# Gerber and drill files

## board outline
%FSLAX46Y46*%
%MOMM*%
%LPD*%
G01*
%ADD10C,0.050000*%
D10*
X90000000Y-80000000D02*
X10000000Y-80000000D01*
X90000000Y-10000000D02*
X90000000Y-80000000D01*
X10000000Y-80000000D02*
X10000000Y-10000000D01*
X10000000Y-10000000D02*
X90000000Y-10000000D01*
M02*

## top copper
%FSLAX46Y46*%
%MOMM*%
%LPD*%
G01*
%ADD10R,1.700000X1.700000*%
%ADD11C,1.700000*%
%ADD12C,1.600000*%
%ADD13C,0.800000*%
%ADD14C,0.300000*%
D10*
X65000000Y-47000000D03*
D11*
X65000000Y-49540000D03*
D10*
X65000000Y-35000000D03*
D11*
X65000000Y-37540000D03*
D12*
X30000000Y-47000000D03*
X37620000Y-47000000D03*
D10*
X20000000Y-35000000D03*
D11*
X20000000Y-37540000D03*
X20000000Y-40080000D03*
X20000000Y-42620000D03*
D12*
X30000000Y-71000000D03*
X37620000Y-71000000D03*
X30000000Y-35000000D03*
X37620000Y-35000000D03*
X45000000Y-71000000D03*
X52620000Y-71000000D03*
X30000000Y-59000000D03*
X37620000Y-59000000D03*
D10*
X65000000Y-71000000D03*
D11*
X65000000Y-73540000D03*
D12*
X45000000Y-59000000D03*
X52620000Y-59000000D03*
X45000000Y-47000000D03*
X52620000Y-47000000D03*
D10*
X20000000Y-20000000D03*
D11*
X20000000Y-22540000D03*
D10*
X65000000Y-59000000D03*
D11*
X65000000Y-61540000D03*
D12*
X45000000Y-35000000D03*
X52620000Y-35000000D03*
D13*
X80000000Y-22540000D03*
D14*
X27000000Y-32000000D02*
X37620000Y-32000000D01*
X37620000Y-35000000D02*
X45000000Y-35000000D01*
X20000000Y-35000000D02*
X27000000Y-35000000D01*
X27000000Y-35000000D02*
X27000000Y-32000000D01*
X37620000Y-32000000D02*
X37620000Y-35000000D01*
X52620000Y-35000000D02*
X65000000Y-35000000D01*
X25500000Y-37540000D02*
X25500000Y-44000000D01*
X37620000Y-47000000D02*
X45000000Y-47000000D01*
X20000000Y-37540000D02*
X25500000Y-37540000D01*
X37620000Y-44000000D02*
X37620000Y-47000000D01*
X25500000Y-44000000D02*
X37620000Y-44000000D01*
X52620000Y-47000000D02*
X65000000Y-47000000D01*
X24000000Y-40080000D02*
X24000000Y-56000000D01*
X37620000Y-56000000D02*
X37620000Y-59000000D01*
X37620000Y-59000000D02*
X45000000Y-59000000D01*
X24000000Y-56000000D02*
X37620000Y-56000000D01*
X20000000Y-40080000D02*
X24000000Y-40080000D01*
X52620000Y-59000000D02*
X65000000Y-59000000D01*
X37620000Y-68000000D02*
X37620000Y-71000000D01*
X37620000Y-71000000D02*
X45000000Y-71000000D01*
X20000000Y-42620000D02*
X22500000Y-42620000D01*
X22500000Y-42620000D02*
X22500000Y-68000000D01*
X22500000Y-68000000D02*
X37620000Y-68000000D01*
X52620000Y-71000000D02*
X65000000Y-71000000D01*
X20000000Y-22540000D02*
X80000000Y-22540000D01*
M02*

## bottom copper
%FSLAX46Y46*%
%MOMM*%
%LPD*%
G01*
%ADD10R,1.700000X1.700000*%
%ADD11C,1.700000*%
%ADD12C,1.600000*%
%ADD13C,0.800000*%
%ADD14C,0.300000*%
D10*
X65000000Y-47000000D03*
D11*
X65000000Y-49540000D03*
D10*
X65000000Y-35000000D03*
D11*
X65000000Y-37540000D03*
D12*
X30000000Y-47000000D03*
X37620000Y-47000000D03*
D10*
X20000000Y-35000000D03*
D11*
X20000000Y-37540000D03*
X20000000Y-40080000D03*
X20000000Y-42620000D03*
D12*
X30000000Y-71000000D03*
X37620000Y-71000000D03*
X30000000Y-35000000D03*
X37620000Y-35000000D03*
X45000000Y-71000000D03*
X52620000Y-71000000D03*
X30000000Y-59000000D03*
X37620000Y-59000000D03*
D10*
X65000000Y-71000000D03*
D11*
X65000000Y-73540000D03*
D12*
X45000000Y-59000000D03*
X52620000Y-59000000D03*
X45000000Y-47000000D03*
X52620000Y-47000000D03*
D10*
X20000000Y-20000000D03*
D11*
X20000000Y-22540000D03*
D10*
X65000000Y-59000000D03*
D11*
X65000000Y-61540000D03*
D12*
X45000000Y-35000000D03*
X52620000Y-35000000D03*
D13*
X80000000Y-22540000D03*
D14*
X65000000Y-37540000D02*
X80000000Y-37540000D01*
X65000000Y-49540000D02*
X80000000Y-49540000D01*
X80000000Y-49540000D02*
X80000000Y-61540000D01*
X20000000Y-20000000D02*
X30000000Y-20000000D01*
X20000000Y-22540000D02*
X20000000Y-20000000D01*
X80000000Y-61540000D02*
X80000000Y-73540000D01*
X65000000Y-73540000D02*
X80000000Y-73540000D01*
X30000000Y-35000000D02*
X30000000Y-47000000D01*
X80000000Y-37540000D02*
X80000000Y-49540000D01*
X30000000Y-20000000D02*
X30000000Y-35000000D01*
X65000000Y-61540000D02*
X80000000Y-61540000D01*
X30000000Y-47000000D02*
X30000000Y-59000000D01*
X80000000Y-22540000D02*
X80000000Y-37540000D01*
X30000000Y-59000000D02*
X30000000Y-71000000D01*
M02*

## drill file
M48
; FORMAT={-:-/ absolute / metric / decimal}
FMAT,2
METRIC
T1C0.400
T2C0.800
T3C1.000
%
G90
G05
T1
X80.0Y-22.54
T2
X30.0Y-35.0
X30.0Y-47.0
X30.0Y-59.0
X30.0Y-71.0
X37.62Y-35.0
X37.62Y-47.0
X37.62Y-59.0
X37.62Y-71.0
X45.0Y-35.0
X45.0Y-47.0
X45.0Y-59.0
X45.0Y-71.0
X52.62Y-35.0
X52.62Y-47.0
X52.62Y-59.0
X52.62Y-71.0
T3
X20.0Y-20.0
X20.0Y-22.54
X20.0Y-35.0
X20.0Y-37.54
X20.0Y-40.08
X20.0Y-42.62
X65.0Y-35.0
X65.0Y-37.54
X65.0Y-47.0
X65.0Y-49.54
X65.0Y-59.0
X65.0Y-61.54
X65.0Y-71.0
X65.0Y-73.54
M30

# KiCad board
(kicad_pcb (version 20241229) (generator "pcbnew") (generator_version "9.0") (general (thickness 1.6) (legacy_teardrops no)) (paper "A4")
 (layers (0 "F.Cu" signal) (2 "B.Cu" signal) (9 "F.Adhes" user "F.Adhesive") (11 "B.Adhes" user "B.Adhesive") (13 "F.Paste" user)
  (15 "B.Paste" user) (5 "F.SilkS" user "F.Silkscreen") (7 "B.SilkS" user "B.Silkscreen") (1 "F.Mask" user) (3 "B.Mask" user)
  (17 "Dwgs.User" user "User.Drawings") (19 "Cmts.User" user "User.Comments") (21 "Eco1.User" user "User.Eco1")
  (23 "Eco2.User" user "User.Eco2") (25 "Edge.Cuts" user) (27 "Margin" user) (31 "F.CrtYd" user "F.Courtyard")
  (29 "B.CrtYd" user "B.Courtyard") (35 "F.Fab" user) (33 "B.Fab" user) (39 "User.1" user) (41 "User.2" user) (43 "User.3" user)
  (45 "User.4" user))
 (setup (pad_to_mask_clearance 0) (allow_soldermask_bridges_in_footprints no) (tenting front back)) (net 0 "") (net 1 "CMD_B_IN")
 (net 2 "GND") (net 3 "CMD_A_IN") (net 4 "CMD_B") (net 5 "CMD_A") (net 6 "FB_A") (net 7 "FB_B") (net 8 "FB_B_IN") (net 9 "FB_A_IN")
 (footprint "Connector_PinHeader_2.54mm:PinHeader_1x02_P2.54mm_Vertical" (layer "F.Cu") (at 65 47)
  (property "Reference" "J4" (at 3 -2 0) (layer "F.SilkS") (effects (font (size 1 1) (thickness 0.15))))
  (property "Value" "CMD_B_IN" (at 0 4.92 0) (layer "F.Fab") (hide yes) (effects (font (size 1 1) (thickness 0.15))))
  (pad "1" thru_hole rect (at 0 0) (size 1.7 1.7) (drill 1) (layers "*.Cu" "*.Mask") (remove_unused_layers no) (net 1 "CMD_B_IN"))
  (pad "2" thru_hole circle (at 0 2.54) (size 1.7 1.7) (drill 1) (layers "*.Cu" "*.Mask") (remove_unused_layers no) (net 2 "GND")))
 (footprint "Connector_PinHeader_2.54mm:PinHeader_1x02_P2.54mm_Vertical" (layer "F.Cu") (at 65 35)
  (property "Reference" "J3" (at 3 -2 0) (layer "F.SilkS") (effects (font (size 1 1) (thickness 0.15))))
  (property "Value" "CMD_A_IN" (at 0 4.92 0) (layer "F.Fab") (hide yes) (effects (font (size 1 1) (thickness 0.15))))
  (pad "1" thru_hole rect (at 0 0) (size 1.7 1.7) (drill 1) (layers "*.Cu" "*.Mask") (remove_unused_layers no) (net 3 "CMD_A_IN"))
  (pad "2" thru_hole circle (at 0 2.54) (size 1.7 1.7) (drill 1) (layers "*.Cu" "*.Mask") (remove_unused_layers no) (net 2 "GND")))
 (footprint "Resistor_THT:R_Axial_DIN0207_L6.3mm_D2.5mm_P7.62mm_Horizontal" (layer "F.Cu") (at 30 47)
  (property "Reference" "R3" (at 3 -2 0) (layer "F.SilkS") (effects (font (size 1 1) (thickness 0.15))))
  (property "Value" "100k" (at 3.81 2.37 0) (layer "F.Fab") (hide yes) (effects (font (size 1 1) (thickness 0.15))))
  (pad "1" thru_hole circle (at 0 0) (size 1.6 1.6) (drill 0.8) (layers "*.Cu" "*.Mask") (remove_unused_layers no) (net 2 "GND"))
  (pad "2" thru_hole circle (at 7.62 0) (size 1.6 1.6) (drill 0.8) (layers "*.Cu" "*.Mask") (remove_unused_layers no) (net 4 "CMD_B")))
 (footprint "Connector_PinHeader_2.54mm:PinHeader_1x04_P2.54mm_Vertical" (layer "F.Cu") (at 20 35)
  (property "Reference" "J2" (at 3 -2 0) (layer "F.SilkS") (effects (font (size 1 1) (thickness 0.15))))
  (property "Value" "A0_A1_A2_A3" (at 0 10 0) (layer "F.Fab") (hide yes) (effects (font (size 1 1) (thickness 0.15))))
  (pad "1" thru_hole rect (at 0 0) (size 1.7 1.7) (drill 1) (layers "*.Cu" "*.Mask") (remove_unused_layers no) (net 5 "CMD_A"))
  (pad "2" thru_hole circle (at 0 2.54) (size 1.7 1.7) (drill 1) (layers "*.Cu" "*.Mask") (remove_unused_layers no) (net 4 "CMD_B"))
  (pad "3" thru_hole circle (at 0 5.08) (size 1.7 1.7) (drill 1) (layers "*.Cu" "*.Mask") (remove_unused_layers no) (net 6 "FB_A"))
  (pad "4" thru_hole circle (at 0 7.62) (size 1.7 1.7) (drill 1) (layers "*.Cu" "*.Mask") (remove_unused_layers no) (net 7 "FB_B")))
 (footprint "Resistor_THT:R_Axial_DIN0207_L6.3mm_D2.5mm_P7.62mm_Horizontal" (layer "F.Cu") (at 30 71)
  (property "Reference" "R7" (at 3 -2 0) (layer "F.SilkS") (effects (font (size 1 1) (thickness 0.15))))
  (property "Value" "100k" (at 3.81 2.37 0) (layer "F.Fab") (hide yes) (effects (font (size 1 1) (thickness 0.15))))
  (pad "1" thru_hole circle (at 0 0) (size 1.6 1.6) (drill 0.8) (layers "*.Cu" "*.Mask") (remove_unused_layers no) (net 2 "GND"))
  (pad "2" thru_hole circle (at 7.62 0) (size 1.6 1.6) (drill 0.8) (layers "*.Cu" "*.Mask") (remove_unused_layers no) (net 7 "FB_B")))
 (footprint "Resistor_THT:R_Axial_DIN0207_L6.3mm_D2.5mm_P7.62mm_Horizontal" (layer "F.Cu") (at 30 35)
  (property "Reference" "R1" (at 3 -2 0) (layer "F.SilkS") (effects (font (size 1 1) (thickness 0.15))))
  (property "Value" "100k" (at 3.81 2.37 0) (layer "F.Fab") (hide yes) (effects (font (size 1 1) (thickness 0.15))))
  (pad "1" thru_hole circle (at 0 0) (size 1.6 1.6) (drill 0.8) (layers "*.Cu" "*.Mask") (remove_unused_layers no) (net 2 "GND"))
  (pad "2" thru_hole circle (at 7.62 0) (size 1.6 1.6) (drill 0.8) (layers "*.Cu" "*.Mask") (remove_unused_layers no) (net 5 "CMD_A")))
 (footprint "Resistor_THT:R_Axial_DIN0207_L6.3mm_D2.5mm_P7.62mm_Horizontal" (layer "F.Cu") (at 45 71)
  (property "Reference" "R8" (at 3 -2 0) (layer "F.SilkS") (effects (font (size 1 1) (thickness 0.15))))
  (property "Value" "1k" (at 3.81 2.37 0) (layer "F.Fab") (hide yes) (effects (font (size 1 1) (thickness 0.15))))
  (pad "1" thru_hole circle (at 0 0) (size 1.6 1.6) (drill 0.8) (layers "*.Cu" "*.Mask") (remove_unused_layers no) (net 7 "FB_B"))
  (pad "2" thru_hole circle (at 7.62 0) (size 1.6 1.6) (drill 0.8) (layers "*.Cu" "*.Mask") (remove_unused_layers no) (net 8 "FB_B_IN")))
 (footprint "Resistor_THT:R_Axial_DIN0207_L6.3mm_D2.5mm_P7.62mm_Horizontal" (layer "F.Cu") (at 30 59)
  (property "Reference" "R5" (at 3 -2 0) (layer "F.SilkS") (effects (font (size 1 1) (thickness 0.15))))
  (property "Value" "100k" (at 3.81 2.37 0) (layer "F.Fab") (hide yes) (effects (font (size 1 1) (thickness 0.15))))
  (pad "1" thru_hole circle (at 0 0) (size 1.6 1.6) (drill 0.8) (layers "*.Cu" "*.Mask") (remove_unused_layers no) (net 2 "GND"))
  (pad "2" thru_hole circle (at 7.62 0) (size 1.6 1.6) (drill 0.8) (layers "*.Cu" "*.Mask") (remove_unused_layers no) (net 6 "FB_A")))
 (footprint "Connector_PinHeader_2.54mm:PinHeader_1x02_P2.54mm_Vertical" (layer "F.Cu") (at 65 71)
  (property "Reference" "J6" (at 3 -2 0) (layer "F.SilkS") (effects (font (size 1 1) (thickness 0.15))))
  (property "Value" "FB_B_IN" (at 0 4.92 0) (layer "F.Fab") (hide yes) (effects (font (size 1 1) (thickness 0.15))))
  (pad "1" thru_hole rect (at 0 0) (size 1.7 1.7) (drill 1) (layers "*.Cu" "*.Mask") (remove_unused_layers no) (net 8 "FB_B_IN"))
  (pad "2" thru_hole circle (at 0 2.54) (size 1.7 1.7) (drill 1) (layers "*.Cu" "*.Mask") (remove_unused_layers no) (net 2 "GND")))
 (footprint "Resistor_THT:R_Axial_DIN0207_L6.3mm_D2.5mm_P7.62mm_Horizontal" (layer "F.Cu") (at 45 59)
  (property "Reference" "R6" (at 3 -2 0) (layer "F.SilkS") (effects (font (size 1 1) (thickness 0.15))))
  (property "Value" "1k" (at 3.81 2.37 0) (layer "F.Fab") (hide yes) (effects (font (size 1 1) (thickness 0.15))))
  (pad "1" thru_hole circle (at 0 0) (size 1.6 1.6) (drill 0.8) (layers "*.Cu" "*.Mask") (remove_unused_layers no) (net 6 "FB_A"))
  (pad "2" thru_hole circle (at 7.62 0) (size 1.6 1.6) (drill 0.8) (layers "*.Cu" "*.Mask") (remove_unused_layers no) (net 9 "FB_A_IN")))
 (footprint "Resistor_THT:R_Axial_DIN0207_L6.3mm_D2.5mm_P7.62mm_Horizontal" (layer "F.Cu") (at 45 47)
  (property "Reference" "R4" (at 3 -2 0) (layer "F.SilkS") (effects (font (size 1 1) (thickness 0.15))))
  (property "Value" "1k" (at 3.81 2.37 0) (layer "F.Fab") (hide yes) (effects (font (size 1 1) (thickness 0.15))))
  (pad "1" thru_hole circle (at 0 0) (size 1.6 1.6) (drill 0.8) (layers "*.Cu" "*.Mask") (remove_unused_layers no) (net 4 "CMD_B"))
  (pad "2" thru_hole circle (at 7.62 0) (size 1.6 1.6) (drill 0.8) (layers "*.Cu" "*.Mask") (remove_unused_layers no) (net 1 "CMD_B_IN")))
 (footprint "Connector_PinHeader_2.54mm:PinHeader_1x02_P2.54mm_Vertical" (layer "F.Cu") (at 20 20)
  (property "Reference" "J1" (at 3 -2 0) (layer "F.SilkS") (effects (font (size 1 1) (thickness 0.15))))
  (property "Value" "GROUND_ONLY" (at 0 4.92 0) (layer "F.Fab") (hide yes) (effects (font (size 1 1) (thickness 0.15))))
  (pad "1" thru_hole rect (at 0 0) (size 1.7 1.7) (drill 1) (layers "*.Cu" "*.Mask") (remove_unused_layers no) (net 2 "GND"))
  (pad "2" thru_hole circle (at 0 2.54) (size 1.7 1.7) (drill 1) (layers "*.Cu" "*.Mask") (remove_unused_layers no) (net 2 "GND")))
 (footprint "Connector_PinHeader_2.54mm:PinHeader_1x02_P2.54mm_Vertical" (layer "F.Cu") (at 65 59)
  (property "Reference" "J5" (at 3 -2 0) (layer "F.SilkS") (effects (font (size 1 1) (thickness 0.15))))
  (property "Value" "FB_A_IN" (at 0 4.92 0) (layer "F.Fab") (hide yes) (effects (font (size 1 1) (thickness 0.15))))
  (pad "1" thru_hole rect (at 0 0) (size 1.7 1.7) (drill 1) (layers "*.Cu" "*.Mask") (remove_unused_layers no) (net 9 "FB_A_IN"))
  (pad "2" thru_hole circle (at 0 2.54) (size 1.7 1.7) (drill 1) (layers "*.Cu" "*.Mask") (remove_unused_layers no) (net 2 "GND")))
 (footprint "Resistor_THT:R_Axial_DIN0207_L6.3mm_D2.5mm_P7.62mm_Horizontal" (layer "F.Cu") (at 45 35)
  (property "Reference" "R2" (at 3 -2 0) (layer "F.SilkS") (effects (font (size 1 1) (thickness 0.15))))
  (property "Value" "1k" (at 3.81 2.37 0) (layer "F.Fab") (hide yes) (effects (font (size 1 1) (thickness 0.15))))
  (pad "1" thru_hole circle (at 0 0) (size 1.6 1.6) (drill 0.8) (layers "*.Cu" "*.Mask") (remove_unused_layers no) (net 5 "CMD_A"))
  (pad "2" thru_hole circle (at 7.62 0) (size 1.6 1.6) (drill 0.8) (layers "*.Cu" "*.Mask") (remove_unused_layers no) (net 3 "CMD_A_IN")))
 (gr_line (start 90 80) (end 10 80) (stroke (width 0.05) (type default)) (layer "Edge.Cuts"))
 (gr_line (start 90 10) (end 90 80) (stroke (width 0.05) (type default)) (layer "Edge.Cuts"))
 (gr_line (start 10 80) (end 10 10) (stroke (width 0.05) (type default)) (layer "Edge.Cuts"))
 (gr_line (start 10 10) (end 90 10) (stroke (width 0.05) (type default)) (layer "Edge.Cuts"))
 (segment (start 27 32) (end 37.62 32) (width 0.3) (layer "F.Cu") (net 5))
 (segment (start 37.62 35) (end 45 35) (width 0.3) (layer "F.Cu") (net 5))
 (segment (start 20 35) (end 27 35) (width 0.3) (layer "F.Cu") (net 5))
 (segment (start 27 35) (end 27 32) (width 0.3) (layer "F.Cu") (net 5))
 (segment (start 37.62 32) (end 37.62 35) (width 0.3) (layer "F.Cu") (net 5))
 (segment (start 52.62 35) (end 65 35) (width 0.3) (layer "F.Cu") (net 3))
 (segment (start 25.5 37.54) (end 25.5 44) (width 0.3) (layer "F.Cu") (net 4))
 (segment (start 37.62 47) (end 45 47) (width 0.3) (layer "F.Cu") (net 4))
 (segment (start 20 37.54) (end 25.5 37.54) (width 0.3) (layer "F.Cu") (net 4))
 (segment (start 37.62 44) (end 37.62 47) (width 0.3) (layer "F.Cu") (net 4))
 (segment (start 25.5 44) (end 37.62 44) (width 0.3) (layer "F.Cu") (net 4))
 (segment (start 52.62 47) (end 65 47) (width 0.3) (layer "F.Cu") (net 1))
 (segment (start 24 40.08) (end 24 56) (width 0.3) (layer "F.Cu") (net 6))
 (segment (start 37.62 56) (end 37.62 59) (width 0.3) (layer "F.Cu") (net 6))
 (segment (start 37.62 59) (end 45 59) (width 0.3) (layer "F.Cu") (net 6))
 (segment (start 24 56) (end 37.62 56) (width 0.3) (layer "F.Cu") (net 6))
 (segment (start 20 40.08) (end 24 40.08) (width 0.3) (layer "F.Cu") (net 6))
 (segment (start 52.62 59) (end 65 59) (width 0.3) (layer "F.Cu") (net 9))
 (segment (start 37.62 68) (end 37.62 71) (width 0.3) (layer "F.Cu") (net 7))
 (segment (start 37.62 71) (end 45 71) (width 0.3) (layer "F.Cu") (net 7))
 (segment (start 20 42.62) (end 22.5 42.62) (width 0.3) (layer "F.Cu") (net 7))
 (segment (start 22.5 42.62) (end 22.5 68) (width 0.3) (layer "F.Cu") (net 7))
 (segment (start 22.5 68) (end 37.62 68) (width 0.3) (layer "F.Cu") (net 7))
 (segment (start 52.62 71) (end 65 71) (width 0.3) (layer "F.Cu") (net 8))
 (segment (start 20 22.54) (end 80 22.54) (width 0.3) (layer "F.Cu") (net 2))
 (via (at 80 22.54) (size 0.8) (drill 0.4) (layers "F.Cu" "B.Cu") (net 2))
 (segment (start 65 37.54) (end 80 37.54) (width 0.3) (layer "B.Cu") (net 2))
 (segment (start 65 49.54) (end 80 49.54) (width 0.3) (layer "B.Cu") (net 2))
 (segment (start 80 49.54) (end 80 61.54) (width 0.3) (layer "B.Cu") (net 2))
 (segment (start 20 20) (end 30 20) (width 0.3) (layer "B.Cu") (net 2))
 (segment (start 20 22.54) (end 20 20) (width 0.3) (layer "B.Cu") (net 2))
 (segment (start 80 61.54) (end 80 73.54) (width 0.3) (layer "B.Cu") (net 2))
 (segment (start 65 73.54) (end 80 73.54) (width 0.3) (layer "B.Cu") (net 2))
 (segment (start 30 35) (end 30 47) (width 0.3) (layer "B.Cu") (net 2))
 (segment (start 80 37.54) (end 80 49.54) (width 0.3) (layer "B.Cu") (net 2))
 (segment (start 30 20) (end 30 35) (width 0.3) (layer "B.Cu") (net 2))
 (segment (start 65 61.54) (end 80 61.54) (width 0.3) (layer "B.Cu") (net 2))
 (segment (start 30 47) (end 30 59) (width 0.3) (layer "B.Cu") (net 2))
 (segment (start 80 22.54) (end 80 37.54) (width 0.3) (layer "B.Cu") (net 2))
 (segment (start 30 59) (end 30 71) (width 0.3) (layer "B.Cu") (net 2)))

